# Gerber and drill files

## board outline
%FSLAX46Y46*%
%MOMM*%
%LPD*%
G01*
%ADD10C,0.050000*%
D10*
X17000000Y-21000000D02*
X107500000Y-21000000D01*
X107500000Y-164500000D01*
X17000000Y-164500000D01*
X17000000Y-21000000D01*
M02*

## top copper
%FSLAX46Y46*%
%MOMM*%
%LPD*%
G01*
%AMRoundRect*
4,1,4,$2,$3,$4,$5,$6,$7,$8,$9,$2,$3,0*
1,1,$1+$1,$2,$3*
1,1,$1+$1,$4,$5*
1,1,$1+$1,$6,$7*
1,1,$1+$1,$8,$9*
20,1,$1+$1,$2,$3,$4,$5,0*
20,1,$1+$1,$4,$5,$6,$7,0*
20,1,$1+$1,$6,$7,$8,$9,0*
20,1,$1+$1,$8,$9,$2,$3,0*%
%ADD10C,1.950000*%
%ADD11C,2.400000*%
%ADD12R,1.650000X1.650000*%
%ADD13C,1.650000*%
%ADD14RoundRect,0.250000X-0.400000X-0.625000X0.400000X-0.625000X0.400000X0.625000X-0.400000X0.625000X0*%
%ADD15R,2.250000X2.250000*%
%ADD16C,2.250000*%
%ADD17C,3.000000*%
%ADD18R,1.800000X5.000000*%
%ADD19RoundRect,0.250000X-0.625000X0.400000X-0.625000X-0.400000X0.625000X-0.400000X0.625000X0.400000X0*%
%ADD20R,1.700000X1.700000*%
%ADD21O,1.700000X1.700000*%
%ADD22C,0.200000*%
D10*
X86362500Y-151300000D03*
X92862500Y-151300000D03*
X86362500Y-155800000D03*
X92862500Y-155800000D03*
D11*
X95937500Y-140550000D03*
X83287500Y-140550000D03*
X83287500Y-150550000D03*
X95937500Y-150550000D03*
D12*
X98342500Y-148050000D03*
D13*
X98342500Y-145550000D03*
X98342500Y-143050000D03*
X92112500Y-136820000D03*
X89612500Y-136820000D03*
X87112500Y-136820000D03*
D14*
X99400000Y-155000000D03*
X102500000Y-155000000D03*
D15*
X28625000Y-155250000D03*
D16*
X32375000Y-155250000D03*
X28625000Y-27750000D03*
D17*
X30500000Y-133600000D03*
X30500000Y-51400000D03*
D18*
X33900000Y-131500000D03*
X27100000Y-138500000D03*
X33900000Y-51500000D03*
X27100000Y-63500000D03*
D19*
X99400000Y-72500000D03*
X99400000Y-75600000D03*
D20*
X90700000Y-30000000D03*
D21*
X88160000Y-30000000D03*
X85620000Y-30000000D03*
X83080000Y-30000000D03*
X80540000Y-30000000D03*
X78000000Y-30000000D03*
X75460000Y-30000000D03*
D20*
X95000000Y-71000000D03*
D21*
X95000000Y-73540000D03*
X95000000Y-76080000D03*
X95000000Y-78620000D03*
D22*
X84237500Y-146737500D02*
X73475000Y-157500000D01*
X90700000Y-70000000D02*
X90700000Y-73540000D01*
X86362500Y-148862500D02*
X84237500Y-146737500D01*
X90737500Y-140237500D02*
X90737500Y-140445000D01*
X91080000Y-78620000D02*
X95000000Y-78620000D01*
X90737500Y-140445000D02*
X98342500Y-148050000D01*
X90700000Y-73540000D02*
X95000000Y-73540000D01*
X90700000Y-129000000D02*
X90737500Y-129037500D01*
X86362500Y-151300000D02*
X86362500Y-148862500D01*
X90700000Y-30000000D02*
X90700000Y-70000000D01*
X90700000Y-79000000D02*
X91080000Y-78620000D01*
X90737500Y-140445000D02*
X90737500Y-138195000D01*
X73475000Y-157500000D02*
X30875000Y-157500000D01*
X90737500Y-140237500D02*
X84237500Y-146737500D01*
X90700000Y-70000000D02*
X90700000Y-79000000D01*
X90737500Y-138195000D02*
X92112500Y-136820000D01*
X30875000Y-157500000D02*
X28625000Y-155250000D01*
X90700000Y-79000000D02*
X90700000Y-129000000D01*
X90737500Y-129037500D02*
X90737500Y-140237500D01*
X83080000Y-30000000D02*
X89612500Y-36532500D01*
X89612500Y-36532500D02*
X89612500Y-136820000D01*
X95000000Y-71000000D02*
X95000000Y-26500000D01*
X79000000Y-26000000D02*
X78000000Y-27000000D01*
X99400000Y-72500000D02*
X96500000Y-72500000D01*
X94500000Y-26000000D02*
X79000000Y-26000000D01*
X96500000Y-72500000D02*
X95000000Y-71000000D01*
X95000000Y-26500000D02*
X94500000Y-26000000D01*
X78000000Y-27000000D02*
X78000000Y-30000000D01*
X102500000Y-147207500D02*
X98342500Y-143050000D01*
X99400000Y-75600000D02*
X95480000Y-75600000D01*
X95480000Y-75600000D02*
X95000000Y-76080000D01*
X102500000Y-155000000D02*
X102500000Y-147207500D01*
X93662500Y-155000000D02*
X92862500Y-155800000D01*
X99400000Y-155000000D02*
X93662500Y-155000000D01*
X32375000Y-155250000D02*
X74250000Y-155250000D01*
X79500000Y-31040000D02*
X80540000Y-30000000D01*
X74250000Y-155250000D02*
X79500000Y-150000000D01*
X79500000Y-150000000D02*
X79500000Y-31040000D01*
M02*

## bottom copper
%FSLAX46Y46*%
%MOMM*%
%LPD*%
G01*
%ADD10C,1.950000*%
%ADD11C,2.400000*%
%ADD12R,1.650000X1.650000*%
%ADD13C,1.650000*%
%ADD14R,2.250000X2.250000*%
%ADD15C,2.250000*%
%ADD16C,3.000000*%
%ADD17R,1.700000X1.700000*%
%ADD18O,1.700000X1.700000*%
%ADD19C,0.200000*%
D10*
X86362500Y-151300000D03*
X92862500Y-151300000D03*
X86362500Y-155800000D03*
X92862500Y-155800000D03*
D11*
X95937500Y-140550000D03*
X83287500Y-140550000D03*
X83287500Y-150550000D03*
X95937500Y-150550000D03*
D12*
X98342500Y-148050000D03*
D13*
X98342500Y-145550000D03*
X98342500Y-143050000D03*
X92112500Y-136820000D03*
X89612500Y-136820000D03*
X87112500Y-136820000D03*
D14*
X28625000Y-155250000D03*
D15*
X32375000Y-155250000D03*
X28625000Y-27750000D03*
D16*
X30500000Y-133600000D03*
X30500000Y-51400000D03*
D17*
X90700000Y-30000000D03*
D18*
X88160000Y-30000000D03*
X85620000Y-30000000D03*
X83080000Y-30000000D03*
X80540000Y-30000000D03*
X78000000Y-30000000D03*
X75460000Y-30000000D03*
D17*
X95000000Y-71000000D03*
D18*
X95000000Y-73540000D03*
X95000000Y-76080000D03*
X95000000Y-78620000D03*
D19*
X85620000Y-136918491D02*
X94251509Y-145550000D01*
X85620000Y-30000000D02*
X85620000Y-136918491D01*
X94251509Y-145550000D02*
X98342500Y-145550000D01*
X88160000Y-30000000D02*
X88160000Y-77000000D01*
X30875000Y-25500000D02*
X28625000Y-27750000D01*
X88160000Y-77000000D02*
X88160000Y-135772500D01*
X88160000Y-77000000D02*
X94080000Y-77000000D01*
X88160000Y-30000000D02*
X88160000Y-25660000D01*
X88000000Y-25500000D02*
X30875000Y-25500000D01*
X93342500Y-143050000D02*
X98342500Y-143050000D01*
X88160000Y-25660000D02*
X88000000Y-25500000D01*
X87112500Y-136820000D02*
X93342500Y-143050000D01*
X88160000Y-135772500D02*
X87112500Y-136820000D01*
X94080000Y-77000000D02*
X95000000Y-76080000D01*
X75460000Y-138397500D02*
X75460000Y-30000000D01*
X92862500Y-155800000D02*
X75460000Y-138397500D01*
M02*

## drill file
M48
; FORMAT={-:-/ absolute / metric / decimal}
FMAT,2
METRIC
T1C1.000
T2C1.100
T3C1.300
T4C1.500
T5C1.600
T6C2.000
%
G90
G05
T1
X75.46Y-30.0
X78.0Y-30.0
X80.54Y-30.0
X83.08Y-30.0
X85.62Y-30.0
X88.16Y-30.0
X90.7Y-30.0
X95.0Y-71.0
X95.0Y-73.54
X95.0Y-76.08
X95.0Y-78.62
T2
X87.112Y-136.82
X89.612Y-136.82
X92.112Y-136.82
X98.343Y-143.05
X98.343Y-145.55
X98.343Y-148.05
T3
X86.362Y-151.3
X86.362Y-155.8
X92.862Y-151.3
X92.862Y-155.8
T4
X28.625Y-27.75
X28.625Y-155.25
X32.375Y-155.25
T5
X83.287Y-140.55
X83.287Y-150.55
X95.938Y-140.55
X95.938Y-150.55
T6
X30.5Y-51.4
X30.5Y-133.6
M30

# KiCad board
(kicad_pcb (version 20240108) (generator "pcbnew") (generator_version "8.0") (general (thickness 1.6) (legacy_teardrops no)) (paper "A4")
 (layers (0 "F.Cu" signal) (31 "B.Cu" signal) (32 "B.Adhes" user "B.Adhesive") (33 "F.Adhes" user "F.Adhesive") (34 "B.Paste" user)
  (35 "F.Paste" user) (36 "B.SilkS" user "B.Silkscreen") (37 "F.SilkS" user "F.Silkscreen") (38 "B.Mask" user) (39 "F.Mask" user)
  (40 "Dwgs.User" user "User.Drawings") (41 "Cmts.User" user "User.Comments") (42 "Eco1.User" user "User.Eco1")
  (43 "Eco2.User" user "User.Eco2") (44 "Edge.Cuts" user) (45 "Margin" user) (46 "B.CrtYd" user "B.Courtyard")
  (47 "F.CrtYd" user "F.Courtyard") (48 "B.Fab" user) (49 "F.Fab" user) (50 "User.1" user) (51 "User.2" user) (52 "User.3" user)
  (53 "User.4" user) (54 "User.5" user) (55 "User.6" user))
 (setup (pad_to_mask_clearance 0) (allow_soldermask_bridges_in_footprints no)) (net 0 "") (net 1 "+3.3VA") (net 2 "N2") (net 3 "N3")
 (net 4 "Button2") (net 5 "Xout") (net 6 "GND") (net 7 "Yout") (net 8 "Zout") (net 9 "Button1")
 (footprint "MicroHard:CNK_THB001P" (layer "F.Cu") (at 89.6125 145.55)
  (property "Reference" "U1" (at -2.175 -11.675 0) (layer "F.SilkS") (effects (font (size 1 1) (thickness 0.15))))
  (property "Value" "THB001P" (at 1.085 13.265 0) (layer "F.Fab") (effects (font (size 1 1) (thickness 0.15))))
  (pad "A" thru_hole circle (at -3.25 5.75) (size 1.95 1.95) (drill 1.3) (layers "*.Cu" "*.Mask") (remove_unused_layers no) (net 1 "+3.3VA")
   (solder_mask_margin 0.102))
  (pad "B" thru_hole circle (at 3.25 5.75) (size 1.95 1.95) (drill 1.3) (layers "*.Cu" "*.Mask") (remove_unused_layers no) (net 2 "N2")
   (solder_mask_margin 0.102))
  (pad "C" thru_hole circle (at -3.25 10.25) (size 1.95 1.95) (drill 1.3) (layers "*.Cu" "*.Mask") (remove_unused_layers no) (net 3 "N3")
   (solder_mask_margin 0.102))
  (pad "D" thru_hole circle (at 3.25 10.25) (size 1.95 1.95) (drill 1.3) (layers "*.Cu" "*.Mask") (remove_unused_layers no)
   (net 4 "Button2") (solder_mask_margin 0.102))
  (pad "S1" thru_hole circle (at 6.325 -5) (size 2.4 2.4) (drill 1.6) (layers "*.Cu" "*.Mask") (remove_unused_layers no)
   (solder_mask_margin 0.102))
  (pad "S2" thru_hole circle (at -6.325 -5) (size 2.4 2.4) (drill 1.6) (layers "*.Cu" "*.Mask") (remove_unused_layers no)
   (solder_mask_margin 0.102))
  (pad "S3" thru_hole circle (at -6.325 5) (size 2.4 2.4) (drill 1.6) (layers "*.Cu" "*.Mask") (remove_unused_layers no)
   (solder_mask_margin 0.102))
  (pad "S4" thru_hole circle (at 6.325 5) (size 2.4 2.4) (drill 1.6) (layers "*.Cu" "*.Mask") (remove_unused_layers no)
   (solder_mask_margin 0.102))
  (pad "VR1_1" thru_hole rect (at 8.73 2.5) (size 1.65 1.65) (drill 1.1) (layers "*.Cu" "*.Mask") (remove_unused_layers no) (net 1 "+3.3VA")
   (solder_mask_margin 0.102))
  (pad "VR1_2" thru_hole circle (at 8.73 0) (size 1.65 1.65) (drill 1.1) (layers "*.Cu" "*.Mask") (remove_unused_layers no) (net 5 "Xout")
   (solder_mask_margin 0.102))
  (pad "VR1_3" thru_hole circle (at 8.73 -2.5) (size 1.65 1.65) (drill 1.1) (layers "*.Cu" "*.Mask") (remove_unused_layers no) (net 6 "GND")
   (solder_mask_margin 0.102))
  (pad "VR2_1" thru_hole circle (at 2.5 -8.73) (size 1.65 1.65) (drill 1.1) (layers "*.Cu" "*.Mask") (remove_unused_layers no)
   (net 1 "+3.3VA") (solder_mask_margin 0.102))
  (pad "VR2_2" thru_hole circle (at 0 -8.73) (size 1.65 1.65) (drill 1.1) (layers "*.Cu" "*.Mask") (remove_unused_layers no) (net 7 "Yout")
   (solder_mask_margin 0.102))
  (pad "VR2_3" thru_hole circle (at -2.5 -8.73) (size 1.65 1.65) (drill 1.1) (layers "*.Cu" "*.Mask") (remove_unused_layers no)
   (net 6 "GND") (solder_mask_margin 0.102)))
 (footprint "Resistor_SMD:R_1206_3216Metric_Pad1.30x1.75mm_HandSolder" (layer "F.Cu") (at 100.95 155)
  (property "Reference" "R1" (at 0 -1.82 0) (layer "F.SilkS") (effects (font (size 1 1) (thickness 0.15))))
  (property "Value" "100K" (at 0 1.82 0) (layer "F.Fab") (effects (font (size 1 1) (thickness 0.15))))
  (pad "1" smd roundrect (at -1.55 0) (size 1.3 1.75) (layers "F.Cu" "F.Paste" "F.Mask") (roundrect_rratio 0.192308) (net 4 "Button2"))
  (pad "2" smd roundrect (at 1.55 0) (size 1.3 1.75) (layers "F.Cu" "F.Paste" "F.Mask") (roundrect_rratio 0.192308) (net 6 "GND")))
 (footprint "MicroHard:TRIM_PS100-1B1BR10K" (layer "F.Cu") (at 30.5 91.5 90)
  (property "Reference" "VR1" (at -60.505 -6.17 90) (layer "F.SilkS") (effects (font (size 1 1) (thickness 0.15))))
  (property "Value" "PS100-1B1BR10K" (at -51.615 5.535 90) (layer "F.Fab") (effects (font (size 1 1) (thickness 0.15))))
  (pad "1" thru_hole rect (at -63.75 -1.875 90) (size 2.25 2.25) (drill 1.5) (layers "*.Cu" "*.Mask") (remove_unused_layers no)
   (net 1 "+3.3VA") (solder_mask_margin 0.102))
  (pad "2" thru_hole circle (at -63.75 1.875 90) (size 2.25 2.25) (drill 1.5) (layers "*.Cu" "*.Mask") (remove_unused_layers no)
   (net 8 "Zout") (solder_mask_margin 0.102))
  (pad "3" thru_hole circle (at 63.75 -1.875 90) (size 2.25 2.25) (drill 1.5) (layers "*.Cu" "*.Mask") (remove_unused_layers no)
   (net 6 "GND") (solder_mask_margin 0.102))
  (pad "P1" thru_hole circle (at -42.1 0 90) (size 3 3) (drill 2) (layers "*.Cu" "*.Mask") (remove_unused_layers no)
   (solder_mask_margin 0.102))
  (pad "P2" thru_hole circle (at 40.1 0 90) (size 3 3) (drill 2) (layers "*.Cu" "*.Mask") (remove_unused_layers no)
   (solder_mask_margin 0.102))
  (pad "P3" smd rect (at -40 3.4 90) (size 5 1.8) (layers "F.Cu" "F.Paste" "F.Mask") (solder_mask_margin 0.102))
  (pad "P4" smd rect (at -47 -3.4 90) (size 5 1.8) (layers "F.Cu" "F.Paste" "F.Mask") (solder_mask_margin 0.102))
  (pad "P5" smd rect (at 40 3.4 90) (size 5 1.8) (layers "F.Cu" "F.Paste" "F.Mask") (solder_mask_margin 0.102))
  (pad "P6" smd rect (at 28 -3.4 90) (size 5 1.8) (layers "F.Cu" "F.Paste" "F.Mask") (solder_mask_margin 0.102)))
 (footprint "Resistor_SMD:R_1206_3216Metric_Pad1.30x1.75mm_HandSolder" (layer "F.Cu") (at 99.4 74.05 -90)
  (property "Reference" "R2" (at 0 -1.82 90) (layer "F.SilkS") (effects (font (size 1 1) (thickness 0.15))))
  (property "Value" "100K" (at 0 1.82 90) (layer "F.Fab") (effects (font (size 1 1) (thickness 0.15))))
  (pad "1" smd roundrect (at -1.55 0 270) (size 1.3 1.75) (layers "F.Cu" "F.Paste" "F.Mask") (roundrect_rratio 0.192308) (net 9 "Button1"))
  (pad "2" smd roundrect (at 1.55 0 270) (size 1.3 1.75) (layers "F.Cu" "F.Paste" "F.Mask") (roundrect_rratio 0.192308) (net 6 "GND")))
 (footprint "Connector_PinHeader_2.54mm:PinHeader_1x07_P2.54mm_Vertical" (layer "F.Cu") (at 90.7 30 -90)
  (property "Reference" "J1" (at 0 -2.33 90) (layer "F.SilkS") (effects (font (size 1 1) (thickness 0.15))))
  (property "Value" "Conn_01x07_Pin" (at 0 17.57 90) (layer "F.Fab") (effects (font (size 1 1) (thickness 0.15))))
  (pad "1" thru_hole rect (at 0 0 270) (size 1.7 1.7) (drill 1) (layers "*.Cu" "*.Mask") (remove_unused_layers no) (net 1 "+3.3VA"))
  (pad "2" thru_hole oval (at 0 2.54 270) (size 1.7 1.7) (drill 1) (layers "*.Cu" "*.Mask") (remove_unused_layers no) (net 6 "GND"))
  (pad "3" thru_hole oval (at 0 5.08 270) (size 1.7 1.7) (drill 1) (layers "*.Cu" "*.Mask") (remove_unused_layers no) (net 5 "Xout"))
  (pad "4" thru_hole oval (at 0 7.62 270) (size 1.7 1.7) (drill 1) (layers "*.Cu" "*.Mask") (remove_unused_layers no) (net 7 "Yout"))
  (pad "5" thru_hole oval (at 0 10.16 270) (size 1.7 1.7) (drill 1) (layers "*.Cu" "*.Mask") (remove_unused_layers no) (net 8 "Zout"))
  (pad "6" thru_hole oval (at 0 12.7 270) (size 1.7 1.7) (drill 1) (layers "*.Cu" "*.Mask") (remove_unused_layers no) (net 9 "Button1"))
  (pad "7" thru_hole oval (at 0 15.24 270) (size 1.7 1.7) (drill 1) (layers "*.Cu" "*.Mask") (remove_unused_layers no) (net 4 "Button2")))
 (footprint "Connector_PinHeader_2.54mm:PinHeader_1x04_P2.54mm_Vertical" (layer "F.Cu") (at 95 71)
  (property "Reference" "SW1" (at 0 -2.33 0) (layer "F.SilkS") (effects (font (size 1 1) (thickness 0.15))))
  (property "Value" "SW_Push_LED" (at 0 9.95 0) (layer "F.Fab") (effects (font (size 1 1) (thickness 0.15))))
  (pad "1" thru_hole rect (at 0 0) (size 1.7 1.7) (drill 1) (layers "*.Cu" "*.Mask") (remove_unused_layers no) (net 9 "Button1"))
  (pad "2" thru_hole oval (at 0 2.54) (size 1.7 1.7) (drill 1) (layers "*.Cu" "*.Mask") (remove_unused_layers no) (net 1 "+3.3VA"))
  (pad "3" thru_hole oval (at 0 5.08) (size 1.7 1.7) (drill 1) (layers "*.Cu" "*.Mask") (remove_unused_layers no) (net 6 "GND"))
  (pad "4" thru_hole oval (at 0 7.62) (size 1.7 1.7) (drill 1) (layers "*.Cu" "*.Mask") (remove_unused_layers no) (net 1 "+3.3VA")))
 (gr_rect (start 17 21) (end 107.5 164.5) (stroke (width 0.05) (type default)) (fill none) (layer "Edge.Cuts"))
 (segment (start 84.2375 146.7375) (end 73.475 157.5) (width 0.2) (layer "F.Cu") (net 1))
 (segment (start 90.7 70) (end 90.7 73.54) (width 0.2) (layer "F.Cu") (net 1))
 (segment (start 86.3625 148.8625) (end 84.2375 146.7375) (width 0.2) (layer "F.Cu") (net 1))
 (segment (start 90.7375 140.2375) (end 90.7375 140.445) (width 0.2) (layer "F.Cu") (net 1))
 (segment (start 91.08 78.62) (end 95 78.62) (width 0.2) (layer "F.Cu") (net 1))
 (segment (start 90.7375 140.445) (end 98.3425 148.05) (width 0.2) (layer "F.Cu") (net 1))
 (segment (start 90.7 73.54) (end 95 73.54) (width 0.2) (layer "F.Cu") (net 1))
 (segment (start 90.7 129) (end 90.7375 129.0375) (width 0.2) (layer "F.Cu") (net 1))
 (segment (start 86.3625 151.3) (end 86.3625 148.8625) (width 0.2) (layer "F.Cu") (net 1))
 (segment (start 90.7 30) (end 90.7 70) (width 0.2) (layer "F.Cu") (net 1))
 (segment (start 90.7 79) (end 91.08 78.62) (width 0.2) (layer "F.Cu") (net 1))
 (segment (start 90.7375 140.445) (end 90.7375 138.195) (width 0.2) (layer "F.Cu") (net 1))
 (segment (start 73.475 157.5) (end 30.875 157.5) (width 0.2) (layer "F.Cu") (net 1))
 (segment (start 90.7375 140.2375) (end 84.2375 146.7375) (width 0.2) (layer "F.Cu") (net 1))
 (segment (start 90.7 70) (end 90.7 79) (width 0.2) (layer "F.Cu") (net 1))
 (segment (start 90.7375 138.195) (end 92.1125 136.82) (width 0.2) (layer "F.Cu") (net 1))
 (segment (start 30.875 157.5) (end 28.625 155.25) (width 0.2) (layer "F.Cu") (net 1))
 (segment (start 90.7 79) (end 90.7 129) (width 0.2) (layer "F.Cu") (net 1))
 (segment (start 90.7375 129.0375) (end 90.7375 140.2375) (width 0.2) (layer "F.Cu") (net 1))
 (segment (start 83.08 30) (end 89.6125 36.5325) (width 0.2) (layer "F.Cu") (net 7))
 (segment (start 89.6125 36.5325) (end 89.6125 136.82) (width 0.2) (layer "F.Cu") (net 7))
 (segment (start 95 71) (end 95 26.5) (width 0.2) (layer "F.Cu") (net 9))
 (segment (start 79 26) (end 78 27) (width 0.2) (layer "F.Cu") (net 9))
 (segment (start 99.4 72.5) (end 96.5 72.5) (width 0.2) (layer "F.Cu") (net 9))
 (segment (start 94.5 26) (end 79 26) (width 0.2) (layer "F.Cu") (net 9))
 (segment (start 96.5 72.5) (end 95 71) (width 0.2) (layer "F.Cu") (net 9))
 (segment (start 95 26.5) (end 94.5 26) (width 0.2) (layer "F.Cu") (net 9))
 (segment (start 78 27) (end 78 30) (width 0.2) (layer "F.Cu") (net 9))
 (segment (start 85.62 136.918491) (end 94.251509 145.55) (width 0.2) (layer "B.Cu") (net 5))
 (segment (start 85.62 30) (end 85.62 136.918491) (width 0.2) (layer "B.Cu") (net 5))
 (segment (start 94.251509 145.55) (end 98.3425 145.55) (width 0.2) (layer "B.Cu") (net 5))
 (segment (start 102.5 147.2075) (end 98.3425 143.05) (width 0.2) (layer "F.Cu") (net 6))
 (segment (start 99.4 75.6) (end 95.48 75.6) (width 0.2) (layer "F.Cu") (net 6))
 (segment (start 95.48 75.6) (end 95 76.08) (width 0.2) (layer "F.Cu") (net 6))
 (segment (start 102.5 155) (end 102.5 147.2075) (width 0.2) (layer "F.Cu") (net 6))
 (segment (start 88.16 30) (end 88.16 77) (width 0.2) (layer "B.Cu") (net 6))
 (segment (start 30.875 25.5) (end 28.625 27.75) (width 0.2) (layer "B.Cu") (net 6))
 (segment (start 88.16 77) (end 88.16 135.7725) (width 0.2) (layer "B.Cu") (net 6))
 (segment (start 88.16 77) (end 94.08 77) (width 0.2) (layer "B.Cu") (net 6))
 (segment (start 88.16 30) (end 88.16 25.66) (width 0.2) (layer "B.Cu") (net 6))
 (segment (start 88 25.5) (end 30.875 25.5) (width 0.2) (layer "B.Cu") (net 6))
 (segment (start 93.3425 143.05) (end 98.3425 143.05) (width 0.2) (layer "B.Cu") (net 6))
 (segment (start 88.16 25.66) (end 88 25.5) (width 0.2) (layer "B.Cu") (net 6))
 (segment (start 87.1125 136.82) (end 93.3425 143.05) (width 0.2) (layer "B.Cu") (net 6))
 (segment (start 88.16 135.7725) (end 87.1125 136.82) (width 0.2) (layer "B.Cu") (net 6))
 (segment (start 94.08 77) (end 95 76.08) (width 0.2) (layer "B.Cu") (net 6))
 (segment (start 93.6625 155) (end 92.8625 155.8) (width 0.2) (layer "F.Cu") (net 4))
 (segment (start 99.4 155) (end 93.6625 155) (width 0.2) (layer "F.Cu") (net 4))
 (segment (start 75.46 138.3975) (end 75.46 30) (width 0.2) (layer "B.Cu") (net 4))
 (segment (start 92.8625 155.8) (end 75.46 138.3975) (width 0.2) (layer "B.Cu") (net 4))
 (segment (start 32.375 155.25) (end 74.25 155.25) (width 0.2) (layer "F.Cu") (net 8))
 (segment (start 79.5 31.04) (end 80.54 30) (width 0.2) (layer "F.Cu") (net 8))
 (segment (start 74.25 155.25) (end 79.5 150) (width 0.2) (layer "F.Cu") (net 8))
 (segment (start 79.5 150) (end 79.5 31.04) (width 0.2) (layer "F.Cu") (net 8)))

